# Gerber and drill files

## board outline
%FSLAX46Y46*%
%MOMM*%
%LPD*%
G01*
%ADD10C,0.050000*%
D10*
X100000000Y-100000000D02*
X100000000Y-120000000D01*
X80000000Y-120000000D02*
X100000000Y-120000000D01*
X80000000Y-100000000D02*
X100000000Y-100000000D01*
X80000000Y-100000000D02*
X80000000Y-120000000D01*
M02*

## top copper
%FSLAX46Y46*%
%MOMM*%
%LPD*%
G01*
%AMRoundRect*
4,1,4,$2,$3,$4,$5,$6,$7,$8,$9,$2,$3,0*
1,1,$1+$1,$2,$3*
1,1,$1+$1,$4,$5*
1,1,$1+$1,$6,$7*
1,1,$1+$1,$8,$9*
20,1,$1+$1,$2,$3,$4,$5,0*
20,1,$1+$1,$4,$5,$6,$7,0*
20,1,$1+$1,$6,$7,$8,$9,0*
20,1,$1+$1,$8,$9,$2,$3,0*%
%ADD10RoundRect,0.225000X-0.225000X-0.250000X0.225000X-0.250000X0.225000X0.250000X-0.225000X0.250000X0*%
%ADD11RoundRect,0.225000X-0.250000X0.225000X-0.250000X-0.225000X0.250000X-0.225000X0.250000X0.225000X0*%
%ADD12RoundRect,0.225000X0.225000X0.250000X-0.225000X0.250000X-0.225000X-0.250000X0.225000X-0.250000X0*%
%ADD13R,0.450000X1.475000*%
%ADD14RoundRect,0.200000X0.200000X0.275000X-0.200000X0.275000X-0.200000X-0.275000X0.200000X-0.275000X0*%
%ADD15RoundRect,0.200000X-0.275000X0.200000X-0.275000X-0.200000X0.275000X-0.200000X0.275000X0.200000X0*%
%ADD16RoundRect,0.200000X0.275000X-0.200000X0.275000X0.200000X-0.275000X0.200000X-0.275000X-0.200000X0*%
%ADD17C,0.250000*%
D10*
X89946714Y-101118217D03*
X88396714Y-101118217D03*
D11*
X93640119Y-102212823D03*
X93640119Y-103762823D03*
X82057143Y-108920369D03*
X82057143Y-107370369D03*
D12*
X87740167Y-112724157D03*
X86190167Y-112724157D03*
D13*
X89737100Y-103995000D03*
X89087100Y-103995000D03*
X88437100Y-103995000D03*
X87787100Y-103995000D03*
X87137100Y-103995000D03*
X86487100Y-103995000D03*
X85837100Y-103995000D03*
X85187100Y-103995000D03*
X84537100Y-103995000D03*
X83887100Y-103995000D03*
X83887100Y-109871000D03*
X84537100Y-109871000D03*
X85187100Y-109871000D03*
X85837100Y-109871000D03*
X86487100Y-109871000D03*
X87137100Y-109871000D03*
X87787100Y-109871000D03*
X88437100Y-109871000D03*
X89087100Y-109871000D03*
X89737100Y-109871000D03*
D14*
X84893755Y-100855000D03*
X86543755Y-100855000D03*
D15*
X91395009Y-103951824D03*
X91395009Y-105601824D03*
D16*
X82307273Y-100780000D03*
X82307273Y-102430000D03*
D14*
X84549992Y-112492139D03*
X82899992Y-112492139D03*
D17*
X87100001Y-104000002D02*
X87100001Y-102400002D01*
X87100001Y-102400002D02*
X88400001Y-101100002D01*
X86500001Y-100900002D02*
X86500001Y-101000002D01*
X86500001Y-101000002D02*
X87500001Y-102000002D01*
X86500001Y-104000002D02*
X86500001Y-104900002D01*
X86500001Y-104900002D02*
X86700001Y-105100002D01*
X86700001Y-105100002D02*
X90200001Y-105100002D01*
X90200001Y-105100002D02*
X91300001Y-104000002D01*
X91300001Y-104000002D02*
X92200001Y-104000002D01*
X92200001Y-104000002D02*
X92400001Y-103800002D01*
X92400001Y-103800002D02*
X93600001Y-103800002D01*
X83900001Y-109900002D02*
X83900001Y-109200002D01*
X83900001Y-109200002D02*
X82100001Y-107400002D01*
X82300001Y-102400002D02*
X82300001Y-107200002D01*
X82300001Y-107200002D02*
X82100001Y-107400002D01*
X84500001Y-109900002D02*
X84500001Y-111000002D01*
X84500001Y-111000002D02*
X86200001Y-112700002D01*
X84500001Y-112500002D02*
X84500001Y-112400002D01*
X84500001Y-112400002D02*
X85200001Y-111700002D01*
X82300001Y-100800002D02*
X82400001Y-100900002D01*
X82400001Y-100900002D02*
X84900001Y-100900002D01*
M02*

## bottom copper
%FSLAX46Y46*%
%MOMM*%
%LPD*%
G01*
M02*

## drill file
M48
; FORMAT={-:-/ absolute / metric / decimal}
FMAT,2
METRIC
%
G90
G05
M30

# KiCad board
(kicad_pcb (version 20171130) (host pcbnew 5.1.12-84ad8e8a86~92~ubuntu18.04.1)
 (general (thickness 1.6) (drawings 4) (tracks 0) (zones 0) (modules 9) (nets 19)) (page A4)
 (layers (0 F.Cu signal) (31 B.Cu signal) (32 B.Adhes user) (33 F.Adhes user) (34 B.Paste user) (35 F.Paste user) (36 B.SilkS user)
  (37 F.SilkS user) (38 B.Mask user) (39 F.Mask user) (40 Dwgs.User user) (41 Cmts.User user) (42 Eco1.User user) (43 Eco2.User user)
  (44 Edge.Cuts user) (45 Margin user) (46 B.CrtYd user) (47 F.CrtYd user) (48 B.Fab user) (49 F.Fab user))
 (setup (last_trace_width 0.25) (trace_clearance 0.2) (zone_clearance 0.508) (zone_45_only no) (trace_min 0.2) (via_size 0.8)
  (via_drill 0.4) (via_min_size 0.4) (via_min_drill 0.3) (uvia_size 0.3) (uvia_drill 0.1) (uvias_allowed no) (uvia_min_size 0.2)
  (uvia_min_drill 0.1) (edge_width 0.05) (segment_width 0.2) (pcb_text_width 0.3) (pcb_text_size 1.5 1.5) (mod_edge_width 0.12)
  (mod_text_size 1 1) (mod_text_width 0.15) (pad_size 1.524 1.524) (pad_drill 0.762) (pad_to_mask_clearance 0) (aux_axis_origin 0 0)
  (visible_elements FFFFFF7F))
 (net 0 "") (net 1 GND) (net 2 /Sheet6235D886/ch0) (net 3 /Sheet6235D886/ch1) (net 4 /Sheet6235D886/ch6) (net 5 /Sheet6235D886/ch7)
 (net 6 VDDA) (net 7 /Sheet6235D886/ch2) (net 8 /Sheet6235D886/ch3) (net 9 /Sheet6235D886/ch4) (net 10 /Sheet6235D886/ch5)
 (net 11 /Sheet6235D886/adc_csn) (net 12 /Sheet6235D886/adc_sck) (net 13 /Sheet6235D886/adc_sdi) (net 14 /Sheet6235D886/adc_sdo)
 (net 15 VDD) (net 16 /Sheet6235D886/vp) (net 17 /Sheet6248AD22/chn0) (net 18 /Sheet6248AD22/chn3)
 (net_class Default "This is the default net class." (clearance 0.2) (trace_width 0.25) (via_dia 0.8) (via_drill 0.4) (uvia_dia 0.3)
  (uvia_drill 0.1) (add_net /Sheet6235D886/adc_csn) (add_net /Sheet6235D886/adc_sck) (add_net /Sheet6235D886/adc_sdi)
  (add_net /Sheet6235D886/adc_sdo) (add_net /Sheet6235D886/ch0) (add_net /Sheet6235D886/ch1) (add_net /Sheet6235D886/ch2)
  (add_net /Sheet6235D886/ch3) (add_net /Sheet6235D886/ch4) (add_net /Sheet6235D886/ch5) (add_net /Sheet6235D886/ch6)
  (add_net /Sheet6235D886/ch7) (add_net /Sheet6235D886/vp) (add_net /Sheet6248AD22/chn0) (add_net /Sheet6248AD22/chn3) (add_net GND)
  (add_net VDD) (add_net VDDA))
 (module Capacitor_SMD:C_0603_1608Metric (layer F.Cu) (at 89.171714 101.118217)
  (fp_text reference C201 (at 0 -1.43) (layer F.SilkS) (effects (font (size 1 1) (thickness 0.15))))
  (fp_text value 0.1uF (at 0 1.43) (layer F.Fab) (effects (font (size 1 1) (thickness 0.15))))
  (pad 2 smd roundrect (at 0.775 0) (size 0.9 0.95) (layers F.Cu F.Mask F.Paste) (roundrect_rratio 0.25) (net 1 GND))
  (pad 1 smd roundrect (at -0.775 0) (size 0.9 0.95) (layers F.Cu F.Mask F.Paste) (roundrect_rratio 0.25) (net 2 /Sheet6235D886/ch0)))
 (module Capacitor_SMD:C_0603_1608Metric (layer F.Cu) (at 93.640119 102.987823 270.000000)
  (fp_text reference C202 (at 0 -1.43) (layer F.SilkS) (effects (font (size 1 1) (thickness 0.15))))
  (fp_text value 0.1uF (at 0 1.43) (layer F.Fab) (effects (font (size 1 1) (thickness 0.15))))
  (pad 1 smd roundrect (at -0.775 0 270.000000) (size 0.9 0.95) (layers F.Cu F.Mask F.Paste) (roundrect_rratio 0.25) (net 1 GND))
  (pad 2 smd roundrect (at 0.775 0 270.000000) (size 0.9 0.95) (layers F.Cu F.Mask F.Paste) (roundrect_rratio 0.25)
   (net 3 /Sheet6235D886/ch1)))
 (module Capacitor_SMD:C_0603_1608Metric (layer F.Cu) (at 82.057143 108.145369 270.000000)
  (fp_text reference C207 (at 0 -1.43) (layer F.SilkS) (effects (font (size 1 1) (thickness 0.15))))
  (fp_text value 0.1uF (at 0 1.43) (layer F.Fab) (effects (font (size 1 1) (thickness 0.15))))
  (pad 2 smd roundrect (at 0.775 0 270.000000) (size 0.9 0.95) (layers F.Cu F.Mask F.Paste) (roundrect_rratio 0.25) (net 1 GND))
  (pad 1 smd roundrect (at -0.775 0 270.000000) (size 0.9 0.95) (layers F.Cu F.Mask F.Paste) (roundrect_rratio 0.25)
   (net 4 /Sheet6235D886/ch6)))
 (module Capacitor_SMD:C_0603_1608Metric (layer F.Cu) (at 86.965167 112.724157 180.000000)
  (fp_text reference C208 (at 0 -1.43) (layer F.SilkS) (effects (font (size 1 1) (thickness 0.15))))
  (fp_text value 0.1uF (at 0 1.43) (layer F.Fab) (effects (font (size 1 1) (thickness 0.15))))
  (pad 1 smd roundrect (at -0.775 0 180.000000) (size 0.9 0.95) (layers F.Cu F.Mask F.Paste) (roundrect_rratio 0.25) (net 1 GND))
  (pad 2 smd roundrect (at 0.775 0 180.000000) (size 0.9 0.95) (layers F.Cu F.Mask F.Paste) (roundrect_rratio 0.25)
   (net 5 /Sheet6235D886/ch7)))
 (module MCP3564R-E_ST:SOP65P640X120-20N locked (layer F.Cu) (at 86.812100 106.933000 270.000000)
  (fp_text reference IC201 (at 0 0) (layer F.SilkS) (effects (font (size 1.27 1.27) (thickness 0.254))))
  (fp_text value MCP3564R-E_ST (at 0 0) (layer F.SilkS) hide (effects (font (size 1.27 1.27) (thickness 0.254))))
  (pad 1 smd rect (at -2.938 -2.925) (size 0.45 1.475) (layers F.Cu F.Mask F.Paste) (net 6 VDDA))
  (pad 2 smd rect (at -2.938 -2.275) (size 0.45 1.475) (layers F.Cu F.Mask F.Paste) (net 1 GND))
  (pad 3 smd rect (at -2.938 -1.625) (size 0.45 1.475) (layers F.Cu F.Mask F.Paste) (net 1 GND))
  (pad 4 smd rect (at -2.938 -0.975) (size 0.45 1.475) (layers F.Cu F.Mask F.Paste))
  (pad 5 smd rect (at -2.938 -0.325) (size 0.45 1.475) (layers F.Cu F.Mask F.Paste) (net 2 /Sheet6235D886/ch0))
  (pad 6 smd rect (at -2.938 0.325) (size 0.45 1.475) (layers F.Cu F.Mask F.Paste) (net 3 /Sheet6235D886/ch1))
  (pad 7 smd rect (at -2.938 0.975) (size 0.45 1.475) (layers F.Cu F.Mask F.Paste) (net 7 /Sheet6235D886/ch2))
  (pad 8 smd rect (at -2.938 1.625) (size 0.45 1.475) (layers F.Cu F.Mask F.Paste) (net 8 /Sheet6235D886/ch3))
  (pad 9 smd rect (at -2.938 2.275) (size 0.45 1.475) (layers F.Cu F.Mask F.Paste) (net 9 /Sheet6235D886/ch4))
  (pad 10 smd rect (at -2.938 2.925) (size 0.45 1.475) (layers F.Cu F.Mask F.Paste) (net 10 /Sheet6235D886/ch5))
  (pad 11 smd rect (at 2.938 2.925) (size 0.45 1.475) (layers F.Cu F.Mask F.Paste) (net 4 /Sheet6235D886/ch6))
  (pad 12 smd rect (at 2.938 2.275) (size 0.45 1.475) (layers F.Cu F.Mask F.Paste) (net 5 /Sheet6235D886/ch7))
  (pad 13 smd rect (at 2.938 1.625) (size 0.45 1.475) (layers F.Cu F.Mask F.Paste) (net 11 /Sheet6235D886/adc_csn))
  (pad 14 smd rect (at 2.938 0.975) (size 0.45 1.475) (layers F.Cu F.Mask F.Paste) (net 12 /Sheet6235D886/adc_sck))
  (pad 15 smd rect (at 2.938 0.325) (size 0.45 1.475) (layers F.Cu F.Mask F.Paste) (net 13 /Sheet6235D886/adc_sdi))
  (pad 16 smd rect (at 2.938 -0.325) (size 0.45 1.475) (layers F.Cu F.Mask F.Paste) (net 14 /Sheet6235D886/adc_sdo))
  (pad 17 smd rect (at 2.938 -0.975) (size 0.45 1.475) (layers F.Cu F.Mask F.Paste))
  (pad 18 smd rect (at 2.938 -1.625) (size 0.45 1.475) (layers F.Cu F.Mask F.Paste))
  (pad 19 smd rect (at 2.938 -2.275) (size 0.45 1.475) (layers F.Cu F.Mask F.Paste) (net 1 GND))
  (pad 20 smd rect (at 2.938 -2.925) (size 0.45 1.475) (layers F.Cu F.Mask F.Paste) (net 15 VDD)))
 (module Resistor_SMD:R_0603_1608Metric (layer F.Cu) (at 85.718755 100.855000 180.000000)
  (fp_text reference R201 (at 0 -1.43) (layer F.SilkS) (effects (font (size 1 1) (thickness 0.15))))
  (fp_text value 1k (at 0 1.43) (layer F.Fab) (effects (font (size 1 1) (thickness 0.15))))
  (pad 2 smd roundrect (at 0.825 0 180.000000) (size 0.8 0.95) (layers F.Cu F.Mask F.Paste) (roundrect_rratio 0.25)
   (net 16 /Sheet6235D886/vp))
  (pad 1 smd roundrect (at -0.825 0 180.000000) (size 0.8 0.95) (layers F.Cu F.Mask F.Paste) (roundrect_rratio 0.25)
   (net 2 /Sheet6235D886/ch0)))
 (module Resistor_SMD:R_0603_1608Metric (layer F.Cu) (at 91.395009 104.776824 270.000000)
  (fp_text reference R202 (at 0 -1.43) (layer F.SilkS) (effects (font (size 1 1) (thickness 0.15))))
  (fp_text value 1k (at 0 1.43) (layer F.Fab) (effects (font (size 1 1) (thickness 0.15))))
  (pad 1 smd roundrect (at -0.825 0 270.000000) (size 0.8 0.95) (layers F.Cu F.Mask F.Paste) (roundrect_rratio 0.25)
   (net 3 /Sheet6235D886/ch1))
  (pad 2 smd roundrect (at 0.825 0 270.000000) (size 0.8 0.95) (layers F.Cu F.Mask F.Paste) (roundrect_rratio 0.25)
   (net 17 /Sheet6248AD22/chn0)))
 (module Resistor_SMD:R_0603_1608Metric (layer F.Cu) (at 82.307273 101.605000 90.000000)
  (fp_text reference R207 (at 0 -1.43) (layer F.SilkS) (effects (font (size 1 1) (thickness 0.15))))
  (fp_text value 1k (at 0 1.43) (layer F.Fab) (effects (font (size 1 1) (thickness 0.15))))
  (pad 2 smd roundrect (at 0.825 0 90.000000) (size 0.8 0.95) (layers F.Cu F.Mask F.Paste) (roundrect_rratio 0.25)
   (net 16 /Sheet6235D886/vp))
  (pad 1 smd roundrect (at -0.825 0 90.000000) (size 0.8 0.95) (layers F.Cu F.Mask F.Paste) (roundrect_rratio 0.25)
   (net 4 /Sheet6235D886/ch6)))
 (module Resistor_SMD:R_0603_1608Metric (layer F.Cu) (at 83.724992 112.492139 180.000000)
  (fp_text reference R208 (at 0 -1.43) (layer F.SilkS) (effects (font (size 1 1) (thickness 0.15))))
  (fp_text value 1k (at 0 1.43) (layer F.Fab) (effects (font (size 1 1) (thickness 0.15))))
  (pad 1 smd roundrect (at -0.825 0 180.000000) (size 0.8 0.95) (layers F.Cu F.Mask F.Paste) (roundrect_rratio 0.25)
   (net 5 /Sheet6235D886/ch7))
  (pad 2 smd roundrect (at 0.825 0 180.000000) (size 0.8 0.95) (layers F.Cu F.Mask F.Paste) (roundrect_rratio 0.25)
   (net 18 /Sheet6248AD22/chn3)))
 (gr_line (start 100 100) (end 100 120) (layer Edge.Cuts) (width 0.05))
 (gr_line (start 80 120) (end 100 120) (layer Edge.Cuts) (width 0.05))
 (gr_line (start 80 100) (end 100 100) (layer Edge.Cuts) (width 0.05))
 (gr_line (start 80 100) (end 80 120) (layer Edge.Cuts) (width 0.05))
 (segment (start 87.100001 104.000002) (end 87.100001 102.400002) (width 0.250000) (layer F.Cu) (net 2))
 (segment (start 87.100001 102.400002) (end 88.400001 101.100002) (width 0.250000) (layer F.Cu) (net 2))
 (segment (start 86.500001 100.900002) (end 86.500001 101.000002) (width 0.250000) (layer F.Cu) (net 2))
 (segment (start 86.500001 101.000002) (end 87.500001 102.000002) (width 0.250000) (layer F.Cu) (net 2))
 (segment (start 86.500001 104.000002) (end 86.500001 104.900002) (width 0.250000) (layer F.Cu) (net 3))
 (segment (start 86.500001 104.900002) (end 86.700001 105.100002) (width 0.250000) (layer F.Cu) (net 3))
 (segment (start 86.700001 105.100002) (end 90.200001 105.100002) (width 0.250000) (layer F.Cu) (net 3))
 (segment (start 90.200001 105.100002) (end 91.300001 104.000002) (width 0.250000) (layer F.Cu) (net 3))
 (segment (start 91.300001 104.000002) (end 92.200001 104.000002) (width 0.250000) (layer F.Cu) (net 3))
 (segment (start 92.200001 104.000002) (end 92.400001 103.800002) (width 0.250000) (layer F.Cu) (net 3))
 (segment (start 92.400001 103.800002) (end 93.600001 103.800002) (width 0.250000) (layer F.Cu) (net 3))
 (segment (start 83.900001 109.900002) (end 83.900001 109.200002) (width 0.250000) (layer F.Cu) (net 4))
 (segment (start 83.900001 109.200002) (end 82.100001 107.400002) (width 0.250000) (layer F.Cu) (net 4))
 (segment (start 82.300001 102.400002) (end 82.300001 107.200002) (width 0.250000) (layer F.Cu) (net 4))
 (segment (start 82.300001 107.200002) (end 82.100001 107.400002) (width 0.250000) (layer F.Cu) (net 4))
 (segment (start 84.500001 109.900002) (end 84.500001 111.000002) (width 0.250000) (layer F.Cu) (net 5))
 (segment (start 84.500001 111.000002) (end 86.200001 112.700002) (width 0.250000) (layer F.Cu) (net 5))
 (segment (start 84.500001 112.500002) (end 84.500001 112.400002) (width 0.250000) (layer F.Cu) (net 5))
 (segment (start 84.500001 112.400002) (end 85.200001 111.700002) (width 0.250000) (layer F.Cu) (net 5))
 (segment (start 82.300001 100.800002) (end 82.400001 100.900002) (width 0.250000) (layer F.Cu) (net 16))
 (segment (start 82.400001 100.900002) (end 84.900001 100.900002) (width 0.250000) (layer F.Cu) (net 16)))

